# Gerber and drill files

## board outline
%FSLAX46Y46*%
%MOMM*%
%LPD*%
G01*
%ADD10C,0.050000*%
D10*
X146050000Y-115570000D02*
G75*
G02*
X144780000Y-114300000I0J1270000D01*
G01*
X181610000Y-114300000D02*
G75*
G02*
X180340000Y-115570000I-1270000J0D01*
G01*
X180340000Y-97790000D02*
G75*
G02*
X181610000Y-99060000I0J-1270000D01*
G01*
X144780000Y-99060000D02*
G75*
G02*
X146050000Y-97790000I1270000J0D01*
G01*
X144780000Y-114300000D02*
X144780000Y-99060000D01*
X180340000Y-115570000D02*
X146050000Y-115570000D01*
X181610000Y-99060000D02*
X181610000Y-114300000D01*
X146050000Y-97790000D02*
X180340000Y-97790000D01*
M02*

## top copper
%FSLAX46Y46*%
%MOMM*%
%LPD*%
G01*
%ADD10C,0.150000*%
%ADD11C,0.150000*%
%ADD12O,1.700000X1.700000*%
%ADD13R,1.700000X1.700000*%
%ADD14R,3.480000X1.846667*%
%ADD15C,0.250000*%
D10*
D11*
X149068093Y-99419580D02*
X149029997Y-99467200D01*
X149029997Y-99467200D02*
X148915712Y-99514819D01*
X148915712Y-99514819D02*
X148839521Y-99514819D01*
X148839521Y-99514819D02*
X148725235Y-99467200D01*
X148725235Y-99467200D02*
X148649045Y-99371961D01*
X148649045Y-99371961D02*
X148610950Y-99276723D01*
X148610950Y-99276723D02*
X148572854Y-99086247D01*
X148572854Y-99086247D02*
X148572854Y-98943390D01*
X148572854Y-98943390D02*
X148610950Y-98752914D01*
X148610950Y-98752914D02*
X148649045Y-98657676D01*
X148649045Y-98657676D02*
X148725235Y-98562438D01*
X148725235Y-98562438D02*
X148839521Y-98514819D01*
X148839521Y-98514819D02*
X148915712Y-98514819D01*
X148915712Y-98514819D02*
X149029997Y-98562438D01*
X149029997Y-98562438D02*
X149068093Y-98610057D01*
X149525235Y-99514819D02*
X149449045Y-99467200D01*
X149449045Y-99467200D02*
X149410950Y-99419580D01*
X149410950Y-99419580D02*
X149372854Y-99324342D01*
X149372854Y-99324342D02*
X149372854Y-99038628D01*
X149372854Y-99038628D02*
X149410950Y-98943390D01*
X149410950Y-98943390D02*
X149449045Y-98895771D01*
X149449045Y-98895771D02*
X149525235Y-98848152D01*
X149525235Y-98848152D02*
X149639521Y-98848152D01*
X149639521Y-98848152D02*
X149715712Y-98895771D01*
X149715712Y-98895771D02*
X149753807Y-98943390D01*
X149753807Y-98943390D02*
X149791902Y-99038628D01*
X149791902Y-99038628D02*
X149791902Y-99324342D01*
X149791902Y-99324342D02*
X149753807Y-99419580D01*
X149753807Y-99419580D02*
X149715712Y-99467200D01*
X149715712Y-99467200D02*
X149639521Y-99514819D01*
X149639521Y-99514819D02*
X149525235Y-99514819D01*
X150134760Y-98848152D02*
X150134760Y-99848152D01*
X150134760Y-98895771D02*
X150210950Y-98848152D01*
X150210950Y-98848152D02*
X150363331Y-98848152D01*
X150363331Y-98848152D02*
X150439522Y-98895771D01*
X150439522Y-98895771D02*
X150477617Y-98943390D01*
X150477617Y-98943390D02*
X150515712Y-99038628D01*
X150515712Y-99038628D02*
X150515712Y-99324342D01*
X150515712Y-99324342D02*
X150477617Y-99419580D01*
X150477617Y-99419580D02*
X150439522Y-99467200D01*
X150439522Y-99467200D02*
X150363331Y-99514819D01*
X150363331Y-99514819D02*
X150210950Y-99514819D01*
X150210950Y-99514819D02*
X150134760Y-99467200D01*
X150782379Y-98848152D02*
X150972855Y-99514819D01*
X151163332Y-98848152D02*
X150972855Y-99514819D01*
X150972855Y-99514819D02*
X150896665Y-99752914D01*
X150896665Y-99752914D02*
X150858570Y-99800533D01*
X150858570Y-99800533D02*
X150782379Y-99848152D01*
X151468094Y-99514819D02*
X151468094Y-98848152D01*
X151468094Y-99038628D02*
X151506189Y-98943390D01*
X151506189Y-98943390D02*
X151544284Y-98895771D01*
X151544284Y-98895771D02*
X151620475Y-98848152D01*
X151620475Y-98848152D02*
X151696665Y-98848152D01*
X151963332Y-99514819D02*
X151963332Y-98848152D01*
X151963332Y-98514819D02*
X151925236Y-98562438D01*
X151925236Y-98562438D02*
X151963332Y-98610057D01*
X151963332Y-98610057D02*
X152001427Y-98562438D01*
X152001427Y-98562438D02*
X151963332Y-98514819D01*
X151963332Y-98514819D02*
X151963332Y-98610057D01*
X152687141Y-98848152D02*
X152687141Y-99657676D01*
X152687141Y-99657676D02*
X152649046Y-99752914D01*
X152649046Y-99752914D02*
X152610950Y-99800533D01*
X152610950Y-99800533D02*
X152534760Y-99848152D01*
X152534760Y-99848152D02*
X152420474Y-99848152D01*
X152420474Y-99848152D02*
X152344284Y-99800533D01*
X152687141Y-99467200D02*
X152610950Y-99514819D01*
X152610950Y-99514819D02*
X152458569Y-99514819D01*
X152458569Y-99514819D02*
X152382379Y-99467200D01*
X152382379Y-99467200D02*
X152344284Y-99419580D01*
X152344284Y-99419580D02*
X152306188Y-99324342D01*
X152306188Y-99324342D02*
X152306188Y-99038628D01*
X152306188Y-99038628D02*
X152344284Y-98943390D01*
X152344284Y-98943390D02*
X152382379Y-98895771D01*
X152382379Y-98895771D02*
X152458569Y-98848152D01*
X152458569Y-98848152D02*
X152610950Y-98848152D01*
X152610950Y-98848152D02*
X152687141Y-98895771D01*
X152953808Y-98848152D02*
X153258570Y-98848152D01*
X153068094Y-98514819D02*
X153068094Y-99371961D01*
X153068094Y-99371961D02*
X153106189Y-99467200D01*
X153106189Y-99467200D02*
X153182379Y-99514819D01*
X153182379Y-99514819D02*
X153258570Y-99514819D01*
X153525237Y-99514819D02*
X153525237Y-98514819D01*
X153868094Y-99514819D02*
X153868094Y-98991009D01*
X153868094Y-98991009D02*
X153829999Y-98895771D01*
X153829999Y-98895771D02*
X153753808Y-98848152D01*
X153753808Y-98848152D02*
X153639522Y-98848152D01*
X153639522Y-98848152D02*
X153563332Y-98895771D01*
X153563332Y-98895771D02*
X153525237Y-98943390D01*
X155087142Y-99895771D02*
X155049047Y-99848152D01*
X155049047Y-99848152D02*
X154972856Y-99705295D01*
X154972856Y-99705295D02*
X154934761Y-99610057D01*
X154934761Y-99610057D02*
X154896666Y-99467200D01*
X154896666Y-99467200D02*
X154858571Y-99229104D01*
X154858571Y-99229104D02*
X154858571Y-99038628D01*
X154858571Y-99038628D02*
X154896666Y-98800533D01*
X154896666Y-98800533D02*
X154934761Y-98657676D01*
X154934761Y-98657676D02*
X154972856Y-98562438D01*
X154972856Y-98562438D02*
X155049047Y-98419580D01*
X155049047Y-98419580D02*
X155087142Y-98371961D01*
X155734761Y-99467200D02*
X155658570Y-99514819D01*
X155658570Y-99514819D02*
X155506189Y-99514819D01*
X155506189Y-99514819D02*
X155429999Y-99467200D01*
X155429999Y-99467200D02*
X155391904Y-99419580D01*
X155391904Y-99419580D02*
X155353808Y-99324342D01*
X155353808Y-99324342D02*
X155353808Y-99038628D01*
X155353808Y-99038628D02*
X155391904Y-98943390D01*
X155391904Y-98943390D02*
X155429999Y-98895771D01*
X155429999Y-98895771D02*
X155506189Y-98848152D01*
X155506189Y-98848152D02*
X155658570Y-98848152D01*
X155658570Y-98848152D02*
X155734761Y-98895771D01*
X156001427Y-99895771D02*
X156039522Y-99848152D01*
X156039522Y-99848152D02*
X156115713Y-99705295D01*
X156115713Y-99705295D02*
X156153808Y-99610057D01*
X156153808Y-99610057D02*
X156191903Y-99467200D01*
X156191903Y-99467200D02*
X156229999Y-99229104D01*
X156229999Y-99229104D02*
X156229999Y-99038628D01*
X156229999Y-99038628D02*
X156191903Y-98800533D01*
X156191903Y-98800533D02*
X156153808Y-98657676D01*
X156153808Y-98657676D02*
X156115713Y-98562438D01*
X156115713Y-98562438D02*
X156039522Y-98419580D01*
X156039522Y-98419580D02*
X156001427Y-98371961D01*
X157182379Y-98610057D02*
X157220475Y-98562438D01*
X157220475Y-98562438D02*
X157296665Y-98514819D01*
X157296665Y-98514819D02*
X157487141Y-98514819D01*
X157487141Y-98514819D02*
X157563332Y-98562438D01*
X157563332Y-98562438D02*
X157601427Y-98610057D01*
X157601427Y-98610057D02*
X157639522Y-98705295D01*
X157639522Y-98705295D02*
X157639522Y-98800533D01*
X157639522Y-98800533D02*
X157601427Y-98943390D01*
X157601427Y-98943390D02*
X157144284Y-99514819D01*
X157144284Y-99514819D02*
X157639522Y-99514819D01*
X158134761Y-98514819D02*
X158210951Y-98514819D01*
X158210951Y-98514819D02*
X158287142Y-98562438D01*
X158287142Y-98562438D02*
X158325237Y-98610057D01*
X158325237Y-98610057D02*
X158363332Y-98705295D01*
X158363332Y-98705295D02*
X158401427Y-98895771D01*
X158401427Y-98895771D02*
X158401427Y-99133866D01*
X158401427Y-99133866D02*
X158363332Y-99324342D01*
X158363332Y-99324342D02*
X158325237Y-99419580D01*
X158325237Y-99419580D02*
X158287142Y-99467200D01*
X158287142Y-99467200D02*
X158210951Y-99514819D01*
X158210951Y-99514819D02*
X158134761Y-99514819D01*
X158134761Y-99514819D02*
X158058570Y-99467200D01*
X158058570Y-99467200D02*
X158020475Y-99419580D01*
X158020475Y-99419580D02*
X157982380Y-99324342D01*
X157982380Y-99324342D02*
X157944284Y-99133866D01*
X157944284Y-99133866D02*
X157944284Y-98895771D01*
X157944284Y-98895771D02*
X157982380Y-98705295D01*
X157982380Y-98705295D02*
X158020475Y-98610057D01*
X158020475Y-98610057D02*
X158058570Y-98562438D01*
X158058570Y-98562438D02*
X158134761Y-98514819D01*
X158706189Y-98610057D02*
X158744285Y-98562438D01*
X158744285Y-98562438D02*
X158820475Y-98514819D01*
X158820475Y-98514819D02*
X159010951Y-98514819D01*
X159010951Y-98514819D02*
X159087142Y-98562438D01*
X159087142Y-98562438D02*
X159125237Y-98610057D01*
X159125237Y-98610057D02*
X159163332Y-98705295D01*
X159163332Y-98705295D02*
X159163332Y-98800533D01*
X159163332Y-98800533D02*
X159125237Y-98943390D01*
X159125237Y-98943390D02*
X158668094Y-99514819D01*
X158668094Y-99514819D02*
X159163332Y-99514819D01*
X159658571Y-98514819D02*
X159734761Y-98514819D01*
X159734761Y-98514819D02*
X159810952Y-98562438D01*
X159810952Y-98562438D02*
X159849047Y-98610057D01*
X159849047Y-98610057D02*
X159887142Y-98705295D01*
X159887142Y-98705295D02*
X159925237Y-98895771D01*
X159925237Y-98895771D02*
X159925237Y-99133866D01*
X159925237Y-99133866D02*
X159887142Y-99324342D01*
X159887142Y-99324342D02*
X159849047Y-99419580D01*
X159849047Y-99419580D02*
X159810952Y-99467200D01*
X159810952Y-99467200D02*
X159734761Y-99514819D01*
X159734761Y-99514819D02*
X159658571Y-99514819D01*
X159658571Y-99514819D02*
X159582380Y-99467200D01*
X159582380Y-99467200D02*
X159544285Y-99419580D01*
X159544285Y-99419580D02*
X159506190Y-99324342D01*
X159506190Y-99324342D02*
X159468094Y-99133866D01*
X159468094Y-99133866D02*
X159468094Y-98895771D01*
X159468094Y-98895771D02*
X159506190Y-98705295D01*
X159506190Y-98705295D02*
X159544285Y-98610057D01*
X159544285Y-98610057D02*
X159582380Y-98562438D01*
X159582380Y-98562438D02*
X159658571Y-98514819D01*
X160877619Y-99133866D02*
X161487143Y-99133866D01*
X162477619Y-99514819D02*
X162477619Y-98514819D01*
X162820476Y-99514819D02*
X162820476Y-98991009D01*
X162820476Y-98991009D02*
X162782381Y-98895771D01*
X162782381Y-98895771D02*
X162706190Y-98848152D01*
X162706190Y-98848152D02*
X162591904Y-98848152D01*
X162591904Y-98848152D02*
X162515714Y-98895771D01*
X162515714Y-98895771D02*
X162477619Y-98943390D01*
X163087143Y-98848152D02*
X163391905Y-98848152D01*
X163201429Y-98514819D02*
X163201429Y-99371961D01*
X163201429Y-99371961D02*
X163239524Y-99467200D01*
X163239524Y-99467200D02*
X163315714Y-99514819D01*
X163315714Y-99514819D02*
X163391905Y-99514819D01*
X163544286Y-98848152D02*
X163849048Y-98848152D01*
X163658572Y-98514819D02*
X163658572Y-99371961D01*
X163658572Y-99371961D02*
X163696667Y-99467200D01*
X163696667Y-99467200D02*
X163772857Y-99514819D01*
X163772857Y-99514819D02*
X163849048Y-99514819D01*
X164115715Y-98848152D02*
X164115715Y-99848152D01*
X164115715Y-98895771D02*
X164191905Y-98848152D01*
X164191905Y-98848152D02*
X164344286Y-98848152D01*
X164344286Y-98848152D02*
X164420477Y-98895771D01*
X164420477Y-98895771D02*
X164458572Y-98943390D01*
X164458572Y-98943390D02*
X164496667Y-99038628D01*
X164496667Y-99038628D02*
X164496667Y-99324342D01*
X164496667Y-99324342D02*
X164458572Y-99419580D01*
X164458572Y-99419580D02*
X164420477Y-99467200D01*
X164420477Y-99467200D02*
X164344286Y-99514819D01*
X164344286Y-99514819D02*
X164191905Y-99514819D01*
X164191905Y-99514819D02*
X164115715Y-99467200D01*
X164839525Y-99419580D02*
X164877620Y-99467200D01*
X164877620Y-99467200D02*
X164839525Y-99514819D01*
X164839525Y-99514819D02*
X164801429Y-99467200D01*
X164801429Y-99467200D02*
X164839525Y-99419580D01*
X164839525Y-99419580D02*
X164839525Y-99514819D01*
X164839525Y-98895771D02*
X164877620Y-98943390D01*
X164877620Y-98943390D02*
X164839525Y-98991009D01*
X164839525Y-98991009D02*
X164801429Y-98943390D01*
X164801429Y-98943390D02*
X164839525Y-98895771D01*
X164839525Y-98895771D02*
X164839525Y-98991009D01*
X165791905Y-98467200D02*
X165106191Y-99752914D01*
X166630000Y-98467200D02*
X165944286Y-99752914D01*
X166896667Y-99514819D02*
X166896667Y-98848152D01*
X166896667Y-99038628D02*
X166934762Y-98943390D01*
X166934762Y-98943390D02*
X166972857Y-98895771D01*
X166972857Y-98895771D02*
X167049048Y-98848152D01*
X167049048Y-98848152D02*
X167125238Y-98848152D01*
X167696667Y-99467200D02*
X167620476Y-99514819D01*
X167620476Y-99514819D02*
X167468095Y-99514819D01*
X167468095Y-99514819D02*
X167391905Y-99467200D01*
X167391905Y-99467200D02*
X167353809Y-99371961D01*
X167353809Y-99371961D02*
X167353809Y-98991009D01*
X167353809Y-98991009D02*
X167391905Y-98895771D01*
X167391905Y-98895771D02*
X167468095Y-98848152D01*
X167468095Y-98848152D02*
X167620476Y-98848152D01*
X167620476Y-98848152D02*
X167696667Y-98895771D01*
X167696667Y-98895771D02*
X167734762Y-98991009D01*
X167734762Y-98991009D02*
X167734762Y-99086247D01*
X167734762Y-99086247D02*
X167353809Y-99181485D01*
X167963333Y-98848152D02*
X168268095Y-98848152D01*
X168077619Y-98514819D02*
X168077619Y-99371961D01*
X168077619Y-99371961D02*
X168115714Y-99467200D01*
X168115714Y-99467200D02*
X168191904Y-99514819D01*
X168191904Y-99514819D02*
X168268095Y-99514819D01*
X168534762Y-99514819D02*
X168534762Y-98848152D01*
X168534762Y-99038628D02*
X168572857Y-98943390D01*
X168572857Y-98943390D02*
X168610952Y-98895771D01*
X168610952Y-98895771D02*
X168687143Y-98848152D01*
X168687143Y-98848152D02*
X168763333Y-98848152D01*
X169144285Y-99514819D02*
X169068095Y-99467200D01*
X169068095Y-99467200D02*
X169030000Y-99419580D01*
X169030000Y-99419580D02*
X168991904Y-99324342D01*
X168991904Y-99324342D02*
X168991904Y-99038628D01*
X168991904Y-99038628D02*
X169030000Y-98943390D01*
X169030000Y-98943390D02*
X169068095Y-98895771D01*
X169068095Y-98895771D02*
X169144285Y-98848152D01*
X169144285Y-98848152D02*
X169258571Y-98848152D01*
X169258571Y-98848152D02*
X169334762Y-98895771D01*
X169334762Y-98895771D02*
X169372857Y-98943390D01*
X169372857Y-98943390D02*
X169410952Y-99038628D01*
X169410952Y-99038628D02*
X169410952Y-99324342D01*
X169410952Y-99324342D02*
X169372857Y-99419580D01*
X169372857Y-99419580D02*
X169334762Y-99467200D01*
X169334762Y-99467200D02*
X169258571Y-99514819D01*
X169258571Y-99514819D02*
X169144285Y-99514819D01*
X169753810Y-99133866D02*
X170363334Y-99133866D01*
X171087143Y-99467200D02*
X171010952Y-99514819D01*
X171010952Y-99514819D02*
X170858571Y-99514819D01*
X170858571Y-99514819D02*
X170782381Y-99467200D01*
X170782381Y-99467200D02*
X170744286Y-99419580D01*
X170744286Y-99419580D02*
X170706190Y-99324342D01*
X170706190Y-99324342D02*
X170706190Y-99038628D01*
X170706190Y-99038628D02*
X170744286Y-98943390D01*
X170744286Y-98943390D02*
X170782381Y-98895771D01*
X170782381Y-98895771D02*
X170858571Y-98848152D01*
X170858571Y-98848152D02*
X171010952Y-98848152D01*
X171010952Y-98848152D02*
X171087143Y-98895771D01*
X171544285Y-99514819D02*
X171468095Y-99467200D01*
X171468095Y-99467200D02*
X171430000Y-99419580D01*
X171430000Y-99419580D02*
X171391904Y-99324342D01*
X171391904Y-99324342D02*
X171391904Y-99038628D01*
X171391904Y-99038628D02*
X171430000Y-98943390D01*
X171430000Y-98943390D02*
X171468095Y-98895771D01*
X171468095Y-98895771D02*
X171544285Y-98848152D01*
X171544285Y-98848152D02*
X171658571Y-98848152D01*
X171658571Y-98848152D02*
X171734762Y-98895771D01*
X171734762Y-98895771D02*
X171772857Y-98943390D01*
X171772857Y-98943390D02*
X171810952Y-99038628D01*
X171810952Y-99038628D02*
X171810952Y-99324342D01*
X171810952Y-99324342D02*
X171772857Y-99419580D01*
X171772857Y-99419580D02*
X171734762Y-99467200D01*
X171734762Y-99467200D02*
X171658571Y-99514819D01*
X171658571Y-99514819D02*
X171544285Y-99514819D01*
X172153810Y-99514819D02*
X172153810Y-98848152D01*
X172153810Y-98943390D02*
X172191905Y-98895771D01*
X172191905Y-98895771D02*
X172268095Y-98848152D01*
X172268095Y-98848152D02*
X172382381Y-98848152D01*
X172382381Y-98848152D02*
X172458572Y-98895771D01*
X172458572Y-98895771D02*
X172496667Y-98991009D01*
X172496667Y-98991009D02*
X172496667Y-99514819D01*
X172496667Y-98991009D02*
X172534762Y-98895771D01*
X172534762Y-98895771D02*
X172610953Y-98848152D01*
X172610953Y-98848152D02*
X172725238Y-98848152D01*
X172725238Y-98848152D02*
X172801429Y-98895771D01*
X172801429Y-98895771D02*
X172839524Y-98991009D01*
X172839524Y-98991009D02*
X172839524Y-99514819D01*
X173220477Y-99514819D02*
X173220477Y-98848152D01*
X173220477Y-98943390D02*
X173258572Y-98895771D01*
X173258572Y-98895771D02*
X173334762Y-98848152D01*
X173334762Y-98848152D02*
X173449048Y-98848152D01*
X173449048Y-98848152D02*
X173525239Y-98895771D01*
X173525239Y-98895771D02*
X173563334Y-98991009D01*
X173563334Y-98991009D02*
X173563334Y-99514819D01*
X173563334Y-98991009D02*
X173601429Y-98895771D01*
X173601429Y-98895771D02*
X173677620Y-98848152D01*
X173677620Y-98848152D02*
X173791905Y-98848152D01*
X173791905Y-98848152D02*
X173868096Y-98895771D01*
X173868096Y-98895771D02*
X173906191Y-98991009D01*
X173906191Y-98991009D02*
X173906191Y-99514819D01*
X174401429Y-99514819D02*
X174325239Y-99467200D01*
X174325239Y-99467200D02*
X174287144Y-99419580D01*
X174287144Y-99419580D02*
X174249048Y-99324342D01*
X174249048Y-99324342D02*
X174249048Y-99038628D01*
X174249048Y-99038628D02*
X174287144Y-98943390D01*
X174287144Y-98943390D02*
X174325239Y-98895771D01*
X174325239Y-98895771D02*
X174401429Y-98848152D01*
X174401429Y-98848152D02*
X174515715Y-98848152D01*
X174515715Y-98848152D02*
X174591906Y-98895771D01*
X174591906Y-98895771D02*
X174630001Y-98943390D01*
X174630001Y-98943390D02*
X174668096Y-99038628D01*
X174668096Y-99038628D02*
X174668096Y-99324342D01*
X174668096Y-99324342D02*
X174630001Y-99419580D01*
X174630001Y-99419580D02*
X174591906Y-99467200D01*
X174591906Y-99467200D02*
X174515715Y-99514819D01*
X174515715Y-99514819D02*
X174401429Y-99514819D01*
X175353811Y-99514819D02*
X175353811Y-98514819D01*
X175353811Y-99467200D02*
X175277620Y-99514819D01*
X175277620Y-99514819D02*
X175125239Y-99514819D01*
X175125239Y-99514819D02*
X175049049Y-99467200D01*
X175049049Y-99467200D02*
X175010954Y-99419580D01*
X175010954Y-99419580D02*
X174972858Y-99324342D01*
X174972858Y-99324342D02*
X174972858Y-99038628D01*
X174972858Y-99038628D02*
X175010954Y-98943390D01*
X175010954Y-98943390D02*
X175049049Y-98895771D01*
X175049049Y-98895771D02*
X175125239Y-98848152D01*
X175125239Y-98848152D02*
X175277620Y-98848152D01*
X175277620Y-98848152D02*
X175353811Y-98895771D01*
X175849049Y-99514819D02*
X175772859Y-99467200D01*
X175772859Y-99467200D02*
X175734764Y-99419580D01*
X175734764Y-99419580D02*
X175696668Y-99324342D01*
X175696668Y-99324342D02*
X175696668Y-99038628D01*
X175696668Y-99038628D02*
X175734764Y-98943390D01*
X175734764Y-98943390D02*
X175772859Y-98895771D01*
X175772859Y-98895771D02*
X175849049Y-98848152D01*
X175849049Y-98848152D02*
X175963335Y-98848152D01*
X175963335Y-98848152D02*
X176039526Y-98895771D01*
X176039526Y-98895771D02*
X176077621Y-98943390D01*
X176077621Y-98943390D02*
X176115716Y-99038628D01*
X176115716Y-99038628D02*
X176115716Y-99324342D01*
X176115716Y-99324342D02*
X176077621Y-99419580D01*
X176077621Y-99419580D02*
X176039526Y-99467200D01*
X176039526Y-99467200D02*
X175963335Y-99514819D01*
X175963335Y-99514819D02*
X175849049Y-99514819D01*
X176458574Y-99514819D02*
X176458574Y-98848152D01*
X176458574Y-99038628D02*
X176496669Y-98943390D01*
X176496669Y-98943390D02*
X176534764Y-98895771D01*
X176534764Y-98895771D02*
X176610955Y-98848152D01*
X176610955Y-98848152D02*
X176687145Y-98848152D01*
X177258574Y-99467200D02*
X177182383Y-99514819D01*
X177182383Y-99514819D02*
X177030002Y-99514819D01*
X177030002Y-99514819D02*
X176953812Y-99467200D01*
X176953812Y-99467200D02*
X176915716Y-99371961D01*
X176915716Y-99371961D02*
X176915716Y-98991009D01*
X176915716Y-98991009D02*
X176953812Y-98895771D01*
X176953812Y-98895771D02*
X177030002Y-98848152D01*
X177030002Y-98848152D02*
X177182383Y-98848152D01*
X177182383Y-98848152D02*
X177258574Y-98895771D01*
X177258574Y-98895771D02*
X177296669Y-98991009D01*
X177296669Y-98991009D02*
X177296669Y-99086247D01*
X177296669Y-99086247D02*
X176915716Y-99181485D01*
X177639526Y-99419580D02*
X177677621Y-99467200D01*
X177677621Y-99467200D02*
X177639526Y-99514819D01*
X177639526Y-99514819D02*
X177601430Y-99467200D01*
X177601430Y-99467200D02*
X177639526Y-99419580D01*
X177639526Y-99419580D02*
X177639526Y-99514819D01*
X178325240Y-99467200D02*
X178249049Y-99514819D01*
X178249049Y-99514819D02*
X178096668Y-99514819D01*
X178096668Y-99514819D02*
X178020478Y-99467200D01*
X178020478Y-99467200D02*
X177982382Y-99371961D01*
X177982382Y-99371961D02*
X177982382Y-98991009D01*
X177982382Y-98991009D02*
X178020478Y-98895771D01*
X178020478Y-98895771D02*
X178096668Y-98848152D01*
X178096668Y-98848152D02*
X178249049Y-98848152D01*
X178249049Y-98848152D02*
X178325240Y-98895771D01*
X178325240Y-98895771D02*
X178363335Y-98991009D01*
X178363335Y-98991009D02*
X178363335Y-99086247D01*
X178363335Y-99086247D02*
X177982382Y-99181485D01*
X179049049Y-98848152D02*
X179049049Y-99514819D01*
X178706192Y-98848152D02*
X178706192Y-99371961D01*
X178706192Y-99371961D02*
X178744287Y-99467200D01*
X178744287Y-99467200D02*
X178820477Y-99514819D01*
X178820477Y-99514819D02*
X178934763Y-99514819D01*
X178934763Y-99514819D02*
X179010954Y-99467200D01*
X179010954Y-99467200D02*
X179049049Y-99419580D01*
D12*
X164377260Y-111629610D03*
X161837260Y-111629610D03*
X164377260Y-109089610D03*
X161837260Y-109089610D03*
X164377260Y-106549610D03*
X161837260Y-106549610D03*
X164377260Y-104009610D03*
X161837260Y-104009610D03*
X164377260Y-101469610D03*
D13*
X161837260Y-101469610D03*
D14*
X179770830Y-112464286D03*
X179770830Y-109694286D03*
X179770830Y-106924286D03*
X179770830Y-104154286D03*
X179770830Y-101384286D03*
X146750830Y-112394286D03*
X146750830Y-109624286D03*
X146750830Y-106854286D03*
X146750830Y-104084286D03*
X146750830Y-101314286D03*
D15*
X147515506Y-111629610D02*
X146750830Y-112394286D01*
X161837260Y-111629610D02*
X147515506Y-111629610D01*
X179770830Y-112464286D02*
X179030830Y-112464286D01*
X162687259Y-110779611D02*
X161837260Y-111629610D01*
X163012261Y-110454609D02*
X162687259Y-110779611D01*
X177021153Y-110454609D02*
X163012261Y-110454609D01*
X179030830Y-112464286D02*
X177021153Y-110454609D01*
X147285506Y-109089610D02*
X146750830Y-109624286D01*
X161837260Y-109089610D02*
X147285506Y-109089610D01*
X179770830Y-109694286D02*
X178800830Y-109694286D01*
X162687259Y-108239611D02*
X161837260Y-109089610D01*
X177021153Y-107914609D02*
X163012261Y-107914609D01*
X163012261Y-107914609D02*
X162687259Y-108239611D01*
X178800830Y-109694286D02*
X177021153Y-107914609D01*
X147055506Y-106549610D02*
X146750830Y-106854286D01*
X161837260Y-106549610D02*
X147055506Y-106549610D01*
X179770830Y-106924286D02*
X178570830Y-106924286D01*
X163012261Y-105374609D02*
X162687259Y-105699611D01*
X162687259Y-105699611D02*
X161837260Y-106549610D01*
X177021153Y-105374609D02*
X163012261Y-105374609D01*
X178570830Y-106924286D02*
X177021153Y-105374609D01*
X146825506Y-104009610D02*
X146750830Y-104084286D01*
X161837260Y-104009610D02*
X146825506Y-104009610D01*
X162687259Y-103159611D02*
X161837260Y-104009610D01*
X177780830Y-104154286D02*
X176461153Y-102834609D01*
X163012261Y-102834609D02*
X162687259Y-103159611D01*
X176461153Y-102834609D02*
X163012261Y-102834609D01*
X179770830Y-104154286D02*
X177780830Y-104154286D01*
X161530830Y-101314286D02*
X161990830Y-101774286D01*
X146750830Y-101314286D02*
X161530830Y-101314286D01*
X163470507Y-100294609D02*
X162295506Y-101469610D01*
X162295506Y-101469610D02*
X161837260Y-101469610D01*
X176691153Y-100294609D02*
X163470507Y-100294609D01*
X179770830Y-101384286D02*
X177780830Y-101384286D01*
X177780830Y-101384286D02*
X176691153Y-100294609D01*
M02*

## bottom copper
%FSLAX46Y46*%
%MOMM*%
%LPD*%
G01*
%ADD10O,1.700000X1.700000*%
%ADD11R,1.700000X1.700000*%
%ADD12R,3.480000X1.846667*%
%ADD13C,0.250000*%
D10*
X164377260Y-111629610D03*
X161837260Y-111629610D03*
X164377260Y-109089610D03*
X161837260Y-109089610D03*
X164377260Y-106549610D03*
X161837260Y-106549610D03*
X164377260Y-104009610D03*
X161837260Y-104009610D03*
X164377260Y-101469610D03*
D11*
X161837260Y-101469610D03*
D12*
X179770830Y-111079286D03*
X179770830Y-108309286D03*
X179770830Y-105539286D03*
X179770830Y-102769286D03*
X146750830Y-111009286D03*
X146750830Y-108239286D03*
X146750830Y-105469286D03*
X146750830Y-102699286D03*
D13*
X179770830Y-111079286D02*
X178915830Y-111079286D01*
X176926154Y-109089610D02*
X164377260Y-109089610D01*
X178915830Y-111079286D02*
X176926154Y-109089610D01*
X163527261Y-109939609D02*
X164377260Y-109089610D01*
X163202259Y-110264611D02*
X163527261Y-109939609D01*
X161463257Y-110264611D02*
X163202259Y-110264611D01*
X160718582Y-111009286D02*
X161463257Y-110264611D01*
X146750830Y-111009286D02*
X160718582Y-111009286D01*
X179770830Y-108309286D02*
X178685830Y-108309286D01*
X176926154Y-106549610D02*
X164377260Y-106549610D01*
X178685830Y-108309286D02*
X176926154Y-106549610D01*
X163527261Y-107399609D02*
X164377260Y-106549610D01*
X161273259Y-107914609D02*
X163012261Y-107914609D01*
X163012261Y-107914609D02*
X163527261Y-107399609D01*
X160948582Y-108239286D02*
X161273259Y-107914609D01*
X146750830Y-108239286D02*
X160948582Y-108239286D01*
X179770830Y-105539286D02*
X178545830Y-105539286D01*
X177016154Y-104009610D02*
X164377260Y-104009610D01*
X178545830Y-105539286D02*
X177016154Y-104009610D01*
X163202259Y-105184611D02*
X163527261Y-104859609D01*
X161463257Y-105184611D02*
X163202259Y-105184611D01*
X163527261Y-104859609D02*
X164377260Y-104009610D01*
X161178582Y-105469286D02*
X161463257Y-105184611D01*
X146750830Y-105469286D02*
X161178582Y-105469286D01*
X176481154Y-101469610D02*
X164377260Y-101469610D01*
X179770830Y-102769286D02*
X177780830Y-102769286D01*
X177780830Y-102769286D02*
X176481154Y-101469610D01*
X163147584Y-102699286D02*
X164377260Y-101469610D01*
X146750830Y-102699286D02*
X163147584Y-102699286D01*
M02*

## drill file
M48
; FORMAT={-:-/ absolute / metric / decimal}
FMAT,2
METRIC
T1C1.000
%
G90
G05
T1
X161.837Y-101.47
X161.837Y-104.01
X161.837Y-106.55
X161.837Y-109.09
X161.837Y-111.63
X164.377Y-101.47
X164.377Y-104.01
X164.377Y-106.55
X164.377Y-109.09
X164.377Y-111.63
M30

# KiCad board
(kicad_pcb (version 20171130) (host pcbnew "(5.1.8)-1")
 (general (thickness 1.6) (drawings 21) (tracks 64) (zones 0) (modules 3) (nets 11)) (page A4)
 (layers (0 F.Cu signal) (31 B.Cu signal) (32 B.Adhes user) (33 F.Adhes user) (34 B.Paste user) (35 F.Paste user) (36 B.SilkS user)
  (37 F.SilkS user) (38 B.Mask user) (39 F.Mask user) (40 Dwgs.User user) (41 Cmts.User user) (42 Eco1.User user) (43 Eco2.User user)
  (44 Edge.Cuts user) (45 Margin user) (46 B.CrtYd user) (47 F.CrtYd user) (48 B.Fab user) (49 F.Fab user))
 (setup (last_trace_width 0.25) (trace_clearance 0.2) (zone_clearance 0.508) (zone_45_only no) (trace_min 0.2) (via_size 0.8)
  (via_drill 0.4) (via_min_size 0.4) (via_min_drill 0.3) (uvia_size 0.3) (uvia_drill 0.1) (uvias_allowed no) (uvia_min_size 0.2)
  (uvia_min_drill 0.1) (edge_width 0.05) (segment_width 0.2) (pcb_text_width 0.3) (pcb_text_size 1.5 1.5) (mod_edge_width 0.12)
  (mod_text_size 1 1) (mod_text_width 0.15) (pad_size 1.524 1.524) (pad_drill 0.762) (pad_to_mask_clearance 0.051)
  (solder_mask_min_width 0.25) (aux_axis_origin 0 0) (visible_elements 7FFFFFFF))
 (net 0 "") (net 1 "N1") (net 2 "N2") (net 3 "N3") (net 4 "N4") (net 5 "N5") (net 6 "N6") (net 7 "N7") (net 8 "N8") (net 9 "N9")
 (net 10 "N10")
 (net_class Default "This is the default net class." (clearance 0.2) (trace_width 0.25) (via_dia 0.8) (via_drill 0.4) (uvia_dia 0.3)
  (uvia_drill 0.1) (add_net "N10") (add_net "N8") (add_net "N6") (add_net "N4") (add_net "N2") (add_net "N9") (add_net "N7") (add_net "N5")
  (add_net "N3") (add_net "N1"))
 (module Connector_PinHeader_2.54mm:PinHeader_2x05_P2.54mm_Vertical (layer F.Cu) (at 161.83726 101.46961)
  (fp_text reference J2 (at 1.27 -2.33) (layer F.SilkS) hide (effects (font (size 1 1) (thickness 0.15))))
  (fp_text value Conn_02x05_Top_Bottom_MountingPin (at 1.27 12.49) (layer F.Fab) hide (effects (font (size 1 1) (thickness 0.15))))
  (pad 10 thru_hole oval (at 2.54 10.16) (size 1.7 1.7) (drill 1) (layers *.Cu *.Mask) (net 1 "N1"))
  (pad 9 thru_hole oval (at 0 10.16) (size 1.7 1.7) (drill 1) (layers *.Cu *.Mask) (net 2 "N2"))
  (pad 8 thru_hole oval (at 2.54 7.62) (size 1.7 1.7) (drill 1) (layers *.Cu *.Mask) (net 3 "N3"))
  (pad 7 thru_hole oval (at 0 7.62) (size 1.7 1.7) (drill 1) (layers *.Cu *.Mask) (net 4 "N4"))
  (pad 6 thru_hole oval (at 2.54 5.08) (size 1.7 1.7) (drill 1) (layers *.Cu *.Mask) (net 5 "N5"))
  (pad 5 thru_hole oval (at 0 5.08) (size 1.7 1.7) (drill 1) (layers *.Cu *.Mask) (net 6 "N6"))
  (pad 4 thru_hole oval (at 2.54 2.54) (size 1.7 1.7) (drill 1) (layers *.Cu *.Mask) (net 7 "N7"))
  (pad 3 thru_hole oval (at 0 2.54) (size 1.7 1.7) (drill 1) (layers *.Cu *.Mask) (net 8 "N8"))
  (pad 2 thru_hole oval (at 2.54 0) (size 1.7 1.7) (drill 1) (layers *.Cu *.Mask) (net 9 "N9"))
  (pad 1 thru_hole rect (at 0 0) (size 1.7 1.7) (drill 1) (layers *.Cu *.Mask) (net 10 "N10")))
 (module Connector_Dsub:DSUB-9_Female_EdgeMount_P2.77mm (layer F.Cu) (at 179.77083 106.924286 90)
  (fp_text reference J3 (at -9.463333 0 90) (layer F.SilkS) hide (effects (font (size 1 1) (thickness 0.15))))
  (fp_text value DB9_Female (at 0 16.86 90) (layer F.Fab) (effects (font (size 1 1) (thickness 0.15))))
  (pad 9 smd rect (at -4.155 0 90) (size 1.846667 3.48) (layers B.Cu B.Paste B.Mask) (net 3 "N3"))
  (pad 8 smd rect (at -1.385 0 90) (size 1.846667 3.48) (layers B.Cu B.Paste B.Mask) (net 5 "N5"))
  (pad 7 smd rect (at 1.385 0 90) (size 1.846667 3.48) (layers B.Cu B.Paste B.Mask) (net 7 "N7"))
  (pad 6 smd rect (at 4.155 0 90) (size 1.846667 3.48) (layers B.Cu B.Paste B.Mask) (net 9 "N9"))
  (pad 5 smd rect (at -5.54 0 90) (size 1.846667 3.48) (layers F.Cu F.Paste F.Mask) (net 2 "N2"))
  (pad 4 smd rect (at -2.77 0 90) (size 1.846667 3.48) (layers F.Cu F.Paste F.Mask) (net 4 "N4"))
  (pad 3 smd rect (at 0 0 90) (size 1.846667 3.48) (layers F.Cu F.Paste F.Mask) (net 6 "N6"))
  (pad 2 smd rect (at 2.77 0 90) (size 1.846667 3.48) (layers F.Cu F.Paste F.Mask) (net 8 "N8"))
  (pad 1 smd rect (at 5.54 0 90) (size 1.846667 3.48) (layers F.Cu F.Paste F.Mask) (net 10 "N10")))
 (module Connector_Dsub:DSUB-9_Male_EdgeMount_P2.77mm (layer F.Cu) (at 146.75083 106.854286 270)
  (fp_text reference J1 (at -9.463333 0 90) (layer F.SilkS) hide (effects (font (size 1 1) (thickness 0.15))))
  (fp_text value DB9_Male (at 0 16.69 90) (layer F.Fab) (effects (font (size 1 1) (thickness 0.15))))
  (pad 9 smd rect (at 4.155 0 270) (size 1.846667 3.48) (layers B.Cu B.Paste B.Mask) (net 3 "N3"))
  (pad 8 smd rect (at 1.385 0 270) (size 1.846667 3.48) (layers B.Cu B.Paste B.Mask) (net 5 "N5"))
  (pad 7 smd rect (at -1.385 0 270) (size 1.846667 3.48) (layers B.Cu B.Paste B.Mask) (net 7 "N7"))
  (pad 6 smd rect (at -4.155 0 270) (size 1.846667 3.48) (layers B.Cu B.Paste B.Mask) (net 9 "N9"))
  (pad 5 smd rect (at 5.54 0 270) (size 1.846667 3.48) (layers F.Cu F.Paste F.Mask) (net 2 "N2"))
  (pad 4 smd rect (at 2.77 0 270) (size 1.846667 3.48) (layers F.Cu F.Paste F.Mask) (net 4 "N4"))
  (pad 3 smd rect (at 0 0 270) (size 1.846667 3.48) (layers F.Cu F.Paste F.Mask) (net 6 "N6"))
  (pad 2 smd rect (at -2.77 0 270) (size 1.846667 3.48) (layers F.Cu F.Paste F.Mask) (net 8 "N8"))
  (pad 1 smd rect (at -5.54 0 270) (size 1.846667 3.48) (layers F.Cu F.Paste F.Mask) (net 10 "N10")))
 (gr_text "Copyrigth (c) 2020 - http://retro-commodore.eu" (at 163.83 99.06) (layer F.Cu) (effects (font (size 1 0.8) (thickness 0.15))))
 (gr_arc (start 146.05 114.3) (end 144.78 114.3) (angle -90) (layer Edge.Cuts) (width 0.05))
 (gr_arc (start 180.34 114.3) (end 180.34 115.57) (angle -90) (layer Edge.Cuts) (width 0.05))
 (gr_arc (start 180.34 99.06) (end 181.61 99.06) (angle -90) (layer Edge.Cuts) (width 0.05))
 (gr_arc (start 146.05 99.06) (end 146.05 97.79) (angle -90) (layer Edge.Cuts) (width 0.05))
 (gr_line (start 144.78 114.3) (end 144.78 99.06) (layer Edge.Cuts) (width 0.05))
 (gr_line (start 180.34 115.57) (end 146.05 115.57) (layer Edge.Cuts) (width 0.05))
 (gr_line (start 181.61 99.06) (end 181.61 114.3) (layer Edge.Cuts) (width 0.05))
 (gr_line (start 146.05 97.79) (end 180.34 97.79) (layer Edge.Cuts) (width 0.05))
 (segment (start 179.77083 111.079286) (end 178.91583 111.079286) (width 0.25) (layer B.Cu) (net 3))
 (segment (start 176.926154 109.08961) (end 164.37726 109.08961) (width 0.25) (layer B.Cu) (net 3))
 (segment (start 178.91583 111.079286) (end 176.926154 109.08961) (width 0.25) (layer B.Cu) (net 3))
 (segment (start 163.527261 109.939609) (end 164.37726 109.08961) (width 0.25) (layer B.Cu) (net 3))
 (segment (start 163.202259 110.264611) (end 163.527261 109.939609) (width 0.25) (layer B.Cu) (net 3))
 (segment (start 161.463257 110.264611) (end 163.202259 110.264611) (width 0.25) (layer B.Cu) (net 3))
 (segment (start 160.718582 111.009286) (end 161.463257 110.264611) (width 0.25) (layer B.Cu) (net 3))
 (segment (start 146.75083 111.009286) (end 160.718582 111.009286) (width 0.25) (layer B.Cu) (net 3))
 (segment (start 179.77083 108.309286) (end 178.68583 108.309286) (width 0.25) (layer B.Cu) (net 5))
 (segment (start 176.926154 106.54961) (end 164.37726 106.54961) (width 0.25) (layer B.Cu) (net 5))
 (segment (start 178.68583 108.309286) (end 176.926154 106.54961) (width 0.25) (layer B.Cu) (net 5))
 (segment (start 163.527261 107.399609) (end 164.37726 106.54961) (width 0.25) (layer B.Cu) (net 5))
 (segment (start 161.273259 107.914609) (end 163.012261 107.914609) (width 0.25) (layer B.Cu) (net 5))
 (segment (start 163.012261 107.914609) (end 163.527261 107.399609) (width 0.25) (layer B.Cu) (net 5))
 (segment (start 160.948582 108.239286) (end 161.273259 107.914609) (width 0.25) (layer B.Cu) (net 5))
 (segment (start 146.75083 108.239286) (end 160.948582 108.239286) (width 0.25) (layer B.Cu) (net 5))
 (segment (start 179.77083 105.539286) (end 178.54583 105.539286) (width 0.25) (layer B.Cu) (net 7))
 (segment (start 177.016154 104.00961) (end 164.37726 104.00961) (width 0.25) (layer B.Cu) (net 7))
 (segment (start 178.54583 105.539286) (end 177.016154 104.00961) (width 0.25) (layer B.Cu) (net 7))
 (segment (start 163.202259 105.184611) (end 163.527261 104.859609) (width 0.25) (layer B.Cu) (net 7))
 (segment (start 161.463257 105.184611) (end 163.202259 105.184611) (width 0.25) (layer B.Cu) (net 7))
 (segment (start 163.527261 104.859609) (end 164.37726 104.00961) (width 0.25) (layer B.Cu) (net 7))
 (segment (start 161.178582 105.469286) (end 161.463257 105.184611) (width 0.25) (layer B.Cu) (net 7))
 (segment (start 146.75083 105.469286) (end 161.178582 105.469286) (width 0.25) (layer B.Cu) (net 7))
 (segment (start 176.481154 101.46961) (end 164.37726 101.46961) (width 0.25) (layer B.Cu) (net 9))
 (segment (start 179.77083 102.769286) (end 177.78083 102.769286) (width 0.25) (layer B.Cu) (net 9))
 (segment (start 177.78083 102.769286) (end 176.481154 101.46961) (width 0.25) (layer B.Cu) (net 9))
 (segment (start 163.147584 102.699286) (end 164.37726 101.46961) (width 0.25) (layer B.Cu) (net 9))
 (segment (start 146.75083 102.699286) (end 163.147584 102.699286) (width 0.25) (layer B.Cu) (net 9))
 (segment (start 147.515506 111.62961) (end 146.75083 112.394286) (width 0.25) (layer F.Cu) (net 2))
 (segment (start 161.83726 111.62961) (end 147.515506 111.62961) (width 0.25) (layer F.Cu) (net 2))
 (segment (start 179.77083 112.464286) (end 179.03083 112.464286) (width 0.25) (layer F.Cu) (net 2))
 (segment (start 162.687259 110.779611) (end 161.83726 111.62961) (width 0.25) (layer F.Cu) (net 2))
 (segment (start 163.012261 110.454609) (end 162.687259 110.779611) (width 0.25) (layer F.Cu) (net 2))
 (segment (start 177.021153 110.454609) (end 163.012261 110.454609) (width 0.25) (layer F.Cu) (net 2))
 (segment (start 179.03083 112.464286) (end 177.021153 110.454609) (width 0.25) (layer F.Cu) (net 2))
 (segment (start 147.285506 109.08961) (end 146.75083 109.624286) (width 0.25) (layer F.Cu) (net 4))
 (segment (start 161.83726 109.08961) (end 147.285506 109.08961) (width 0.25) (layer F.Cu) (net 4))
 (segment (start 179.77083 109.694286) (end 178.80083 109.694286) (width 0.25) (layer F.Cu) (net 4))
 (segment (start 162.687259 108.239611) (end 161.83726 109.08961) (width 0.25) (layer F.Cu) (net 4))
 (segment (start 177.021153 107.914609) (end 163.012261 107.914609) (width 0.25) (layer F.Cu) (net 4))
 (segment (start 163.012261 107.914609) (end 162.687259 108.239611) (width 0.25) (layer F.Cu) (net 4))
 (segment (start 178.80083 109.694286) (end 177.021153 107.914609) (width 0.25) (layer F.Cu) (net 4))
 (segment (start 147.055506 106.54961) (end 146.75083 106.854286) (width 0.25) (layer F.Cu) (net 6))
 (segment (start 161.83726 106.54961) (end 147.055506 106.54961) (width 0.25) (layer F.Cu) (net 6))
 (segment (start 179.77083 106.924286) (end 178.57083 106.924286) (width 0.25) (layer F.Cu) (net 6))
 (segment (start 163.012261 105.374609) (end 162.687259 105.699611) (width 0.25) (layer F.Cu) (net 6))
 (segment (start 162.687259 105.699611) (end 161.83726 106.54961) (width 0.25) (layer F.Cu) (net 6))
 (segment (start 177.021153 105.374609) (end 163.012261 105.374609) (width 0.25) (layer F.Cu) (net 6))
 (segment (start 178.57083 106.924286) (end 177.021153 105.374609) (width 0.25) (layer F.Cu) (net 6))
 (segment (start 146.825506 104.00961) (end 146.75083 104.084286) (width 0.25) (layer F.Cu) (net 8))
 (segment (start 161.83726 104.00961) (end 146.825506 104.00961) (width 0.25) (layer F.Cu) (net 8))
 (segment (start 162.687259 103.159611) (end 161.83726 104.00961) (width 0.25) (layer F.Cu) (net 8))
 (segment (start 177.78083 104.154286) (end 176.461153 102.834609) (width 0.25) (layer F.Cu) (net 8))
 (segment (start 163.012261 102.834609) (end 162.687259 103.159611) (width 0.25) (layer F.Cu) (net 8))
 (segment (start 176.461153 102.834609) (end 163.012261 102.834609) (width 0.25) (layer F.Cu) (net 8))
 (segment (start 179.77083 104.154286) (end 177.78083 104.154286) (width 0.25) (layer F.Cu) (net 8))
 (segment (start 161.53083 101.314286) (end 161.99083 101.774286) (width 0.25) (layer F.Cu) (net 10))
 (segment (start 146.75083 101.314286) (end 161.53083 101.314286) (width 0.25) (layer F.Cu) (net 10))
 (segment (start 163.470507 100.294609) (end 162.295506 101.46961) (width 0.25) (layer F.Cu) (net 10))
 (segment (start 162.295506 101.46961) (end 161.83726 101.46961) (width 0.25) (layer F.Cu) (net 10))
 (segment (start 176.691153 100.294609) (end 163.470507 100.294609) (width 0.25) (layer F.Cu) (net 10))
 (segment (start 179.77083 101.384286) (end 177.78083 101.384286) (width 0.25) (layer F.Cu) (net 10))
 (segment (start 177.78083 101.384286) (end 176.691153 100.294609) (width 0.25) (layer F.Cu) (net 10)))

